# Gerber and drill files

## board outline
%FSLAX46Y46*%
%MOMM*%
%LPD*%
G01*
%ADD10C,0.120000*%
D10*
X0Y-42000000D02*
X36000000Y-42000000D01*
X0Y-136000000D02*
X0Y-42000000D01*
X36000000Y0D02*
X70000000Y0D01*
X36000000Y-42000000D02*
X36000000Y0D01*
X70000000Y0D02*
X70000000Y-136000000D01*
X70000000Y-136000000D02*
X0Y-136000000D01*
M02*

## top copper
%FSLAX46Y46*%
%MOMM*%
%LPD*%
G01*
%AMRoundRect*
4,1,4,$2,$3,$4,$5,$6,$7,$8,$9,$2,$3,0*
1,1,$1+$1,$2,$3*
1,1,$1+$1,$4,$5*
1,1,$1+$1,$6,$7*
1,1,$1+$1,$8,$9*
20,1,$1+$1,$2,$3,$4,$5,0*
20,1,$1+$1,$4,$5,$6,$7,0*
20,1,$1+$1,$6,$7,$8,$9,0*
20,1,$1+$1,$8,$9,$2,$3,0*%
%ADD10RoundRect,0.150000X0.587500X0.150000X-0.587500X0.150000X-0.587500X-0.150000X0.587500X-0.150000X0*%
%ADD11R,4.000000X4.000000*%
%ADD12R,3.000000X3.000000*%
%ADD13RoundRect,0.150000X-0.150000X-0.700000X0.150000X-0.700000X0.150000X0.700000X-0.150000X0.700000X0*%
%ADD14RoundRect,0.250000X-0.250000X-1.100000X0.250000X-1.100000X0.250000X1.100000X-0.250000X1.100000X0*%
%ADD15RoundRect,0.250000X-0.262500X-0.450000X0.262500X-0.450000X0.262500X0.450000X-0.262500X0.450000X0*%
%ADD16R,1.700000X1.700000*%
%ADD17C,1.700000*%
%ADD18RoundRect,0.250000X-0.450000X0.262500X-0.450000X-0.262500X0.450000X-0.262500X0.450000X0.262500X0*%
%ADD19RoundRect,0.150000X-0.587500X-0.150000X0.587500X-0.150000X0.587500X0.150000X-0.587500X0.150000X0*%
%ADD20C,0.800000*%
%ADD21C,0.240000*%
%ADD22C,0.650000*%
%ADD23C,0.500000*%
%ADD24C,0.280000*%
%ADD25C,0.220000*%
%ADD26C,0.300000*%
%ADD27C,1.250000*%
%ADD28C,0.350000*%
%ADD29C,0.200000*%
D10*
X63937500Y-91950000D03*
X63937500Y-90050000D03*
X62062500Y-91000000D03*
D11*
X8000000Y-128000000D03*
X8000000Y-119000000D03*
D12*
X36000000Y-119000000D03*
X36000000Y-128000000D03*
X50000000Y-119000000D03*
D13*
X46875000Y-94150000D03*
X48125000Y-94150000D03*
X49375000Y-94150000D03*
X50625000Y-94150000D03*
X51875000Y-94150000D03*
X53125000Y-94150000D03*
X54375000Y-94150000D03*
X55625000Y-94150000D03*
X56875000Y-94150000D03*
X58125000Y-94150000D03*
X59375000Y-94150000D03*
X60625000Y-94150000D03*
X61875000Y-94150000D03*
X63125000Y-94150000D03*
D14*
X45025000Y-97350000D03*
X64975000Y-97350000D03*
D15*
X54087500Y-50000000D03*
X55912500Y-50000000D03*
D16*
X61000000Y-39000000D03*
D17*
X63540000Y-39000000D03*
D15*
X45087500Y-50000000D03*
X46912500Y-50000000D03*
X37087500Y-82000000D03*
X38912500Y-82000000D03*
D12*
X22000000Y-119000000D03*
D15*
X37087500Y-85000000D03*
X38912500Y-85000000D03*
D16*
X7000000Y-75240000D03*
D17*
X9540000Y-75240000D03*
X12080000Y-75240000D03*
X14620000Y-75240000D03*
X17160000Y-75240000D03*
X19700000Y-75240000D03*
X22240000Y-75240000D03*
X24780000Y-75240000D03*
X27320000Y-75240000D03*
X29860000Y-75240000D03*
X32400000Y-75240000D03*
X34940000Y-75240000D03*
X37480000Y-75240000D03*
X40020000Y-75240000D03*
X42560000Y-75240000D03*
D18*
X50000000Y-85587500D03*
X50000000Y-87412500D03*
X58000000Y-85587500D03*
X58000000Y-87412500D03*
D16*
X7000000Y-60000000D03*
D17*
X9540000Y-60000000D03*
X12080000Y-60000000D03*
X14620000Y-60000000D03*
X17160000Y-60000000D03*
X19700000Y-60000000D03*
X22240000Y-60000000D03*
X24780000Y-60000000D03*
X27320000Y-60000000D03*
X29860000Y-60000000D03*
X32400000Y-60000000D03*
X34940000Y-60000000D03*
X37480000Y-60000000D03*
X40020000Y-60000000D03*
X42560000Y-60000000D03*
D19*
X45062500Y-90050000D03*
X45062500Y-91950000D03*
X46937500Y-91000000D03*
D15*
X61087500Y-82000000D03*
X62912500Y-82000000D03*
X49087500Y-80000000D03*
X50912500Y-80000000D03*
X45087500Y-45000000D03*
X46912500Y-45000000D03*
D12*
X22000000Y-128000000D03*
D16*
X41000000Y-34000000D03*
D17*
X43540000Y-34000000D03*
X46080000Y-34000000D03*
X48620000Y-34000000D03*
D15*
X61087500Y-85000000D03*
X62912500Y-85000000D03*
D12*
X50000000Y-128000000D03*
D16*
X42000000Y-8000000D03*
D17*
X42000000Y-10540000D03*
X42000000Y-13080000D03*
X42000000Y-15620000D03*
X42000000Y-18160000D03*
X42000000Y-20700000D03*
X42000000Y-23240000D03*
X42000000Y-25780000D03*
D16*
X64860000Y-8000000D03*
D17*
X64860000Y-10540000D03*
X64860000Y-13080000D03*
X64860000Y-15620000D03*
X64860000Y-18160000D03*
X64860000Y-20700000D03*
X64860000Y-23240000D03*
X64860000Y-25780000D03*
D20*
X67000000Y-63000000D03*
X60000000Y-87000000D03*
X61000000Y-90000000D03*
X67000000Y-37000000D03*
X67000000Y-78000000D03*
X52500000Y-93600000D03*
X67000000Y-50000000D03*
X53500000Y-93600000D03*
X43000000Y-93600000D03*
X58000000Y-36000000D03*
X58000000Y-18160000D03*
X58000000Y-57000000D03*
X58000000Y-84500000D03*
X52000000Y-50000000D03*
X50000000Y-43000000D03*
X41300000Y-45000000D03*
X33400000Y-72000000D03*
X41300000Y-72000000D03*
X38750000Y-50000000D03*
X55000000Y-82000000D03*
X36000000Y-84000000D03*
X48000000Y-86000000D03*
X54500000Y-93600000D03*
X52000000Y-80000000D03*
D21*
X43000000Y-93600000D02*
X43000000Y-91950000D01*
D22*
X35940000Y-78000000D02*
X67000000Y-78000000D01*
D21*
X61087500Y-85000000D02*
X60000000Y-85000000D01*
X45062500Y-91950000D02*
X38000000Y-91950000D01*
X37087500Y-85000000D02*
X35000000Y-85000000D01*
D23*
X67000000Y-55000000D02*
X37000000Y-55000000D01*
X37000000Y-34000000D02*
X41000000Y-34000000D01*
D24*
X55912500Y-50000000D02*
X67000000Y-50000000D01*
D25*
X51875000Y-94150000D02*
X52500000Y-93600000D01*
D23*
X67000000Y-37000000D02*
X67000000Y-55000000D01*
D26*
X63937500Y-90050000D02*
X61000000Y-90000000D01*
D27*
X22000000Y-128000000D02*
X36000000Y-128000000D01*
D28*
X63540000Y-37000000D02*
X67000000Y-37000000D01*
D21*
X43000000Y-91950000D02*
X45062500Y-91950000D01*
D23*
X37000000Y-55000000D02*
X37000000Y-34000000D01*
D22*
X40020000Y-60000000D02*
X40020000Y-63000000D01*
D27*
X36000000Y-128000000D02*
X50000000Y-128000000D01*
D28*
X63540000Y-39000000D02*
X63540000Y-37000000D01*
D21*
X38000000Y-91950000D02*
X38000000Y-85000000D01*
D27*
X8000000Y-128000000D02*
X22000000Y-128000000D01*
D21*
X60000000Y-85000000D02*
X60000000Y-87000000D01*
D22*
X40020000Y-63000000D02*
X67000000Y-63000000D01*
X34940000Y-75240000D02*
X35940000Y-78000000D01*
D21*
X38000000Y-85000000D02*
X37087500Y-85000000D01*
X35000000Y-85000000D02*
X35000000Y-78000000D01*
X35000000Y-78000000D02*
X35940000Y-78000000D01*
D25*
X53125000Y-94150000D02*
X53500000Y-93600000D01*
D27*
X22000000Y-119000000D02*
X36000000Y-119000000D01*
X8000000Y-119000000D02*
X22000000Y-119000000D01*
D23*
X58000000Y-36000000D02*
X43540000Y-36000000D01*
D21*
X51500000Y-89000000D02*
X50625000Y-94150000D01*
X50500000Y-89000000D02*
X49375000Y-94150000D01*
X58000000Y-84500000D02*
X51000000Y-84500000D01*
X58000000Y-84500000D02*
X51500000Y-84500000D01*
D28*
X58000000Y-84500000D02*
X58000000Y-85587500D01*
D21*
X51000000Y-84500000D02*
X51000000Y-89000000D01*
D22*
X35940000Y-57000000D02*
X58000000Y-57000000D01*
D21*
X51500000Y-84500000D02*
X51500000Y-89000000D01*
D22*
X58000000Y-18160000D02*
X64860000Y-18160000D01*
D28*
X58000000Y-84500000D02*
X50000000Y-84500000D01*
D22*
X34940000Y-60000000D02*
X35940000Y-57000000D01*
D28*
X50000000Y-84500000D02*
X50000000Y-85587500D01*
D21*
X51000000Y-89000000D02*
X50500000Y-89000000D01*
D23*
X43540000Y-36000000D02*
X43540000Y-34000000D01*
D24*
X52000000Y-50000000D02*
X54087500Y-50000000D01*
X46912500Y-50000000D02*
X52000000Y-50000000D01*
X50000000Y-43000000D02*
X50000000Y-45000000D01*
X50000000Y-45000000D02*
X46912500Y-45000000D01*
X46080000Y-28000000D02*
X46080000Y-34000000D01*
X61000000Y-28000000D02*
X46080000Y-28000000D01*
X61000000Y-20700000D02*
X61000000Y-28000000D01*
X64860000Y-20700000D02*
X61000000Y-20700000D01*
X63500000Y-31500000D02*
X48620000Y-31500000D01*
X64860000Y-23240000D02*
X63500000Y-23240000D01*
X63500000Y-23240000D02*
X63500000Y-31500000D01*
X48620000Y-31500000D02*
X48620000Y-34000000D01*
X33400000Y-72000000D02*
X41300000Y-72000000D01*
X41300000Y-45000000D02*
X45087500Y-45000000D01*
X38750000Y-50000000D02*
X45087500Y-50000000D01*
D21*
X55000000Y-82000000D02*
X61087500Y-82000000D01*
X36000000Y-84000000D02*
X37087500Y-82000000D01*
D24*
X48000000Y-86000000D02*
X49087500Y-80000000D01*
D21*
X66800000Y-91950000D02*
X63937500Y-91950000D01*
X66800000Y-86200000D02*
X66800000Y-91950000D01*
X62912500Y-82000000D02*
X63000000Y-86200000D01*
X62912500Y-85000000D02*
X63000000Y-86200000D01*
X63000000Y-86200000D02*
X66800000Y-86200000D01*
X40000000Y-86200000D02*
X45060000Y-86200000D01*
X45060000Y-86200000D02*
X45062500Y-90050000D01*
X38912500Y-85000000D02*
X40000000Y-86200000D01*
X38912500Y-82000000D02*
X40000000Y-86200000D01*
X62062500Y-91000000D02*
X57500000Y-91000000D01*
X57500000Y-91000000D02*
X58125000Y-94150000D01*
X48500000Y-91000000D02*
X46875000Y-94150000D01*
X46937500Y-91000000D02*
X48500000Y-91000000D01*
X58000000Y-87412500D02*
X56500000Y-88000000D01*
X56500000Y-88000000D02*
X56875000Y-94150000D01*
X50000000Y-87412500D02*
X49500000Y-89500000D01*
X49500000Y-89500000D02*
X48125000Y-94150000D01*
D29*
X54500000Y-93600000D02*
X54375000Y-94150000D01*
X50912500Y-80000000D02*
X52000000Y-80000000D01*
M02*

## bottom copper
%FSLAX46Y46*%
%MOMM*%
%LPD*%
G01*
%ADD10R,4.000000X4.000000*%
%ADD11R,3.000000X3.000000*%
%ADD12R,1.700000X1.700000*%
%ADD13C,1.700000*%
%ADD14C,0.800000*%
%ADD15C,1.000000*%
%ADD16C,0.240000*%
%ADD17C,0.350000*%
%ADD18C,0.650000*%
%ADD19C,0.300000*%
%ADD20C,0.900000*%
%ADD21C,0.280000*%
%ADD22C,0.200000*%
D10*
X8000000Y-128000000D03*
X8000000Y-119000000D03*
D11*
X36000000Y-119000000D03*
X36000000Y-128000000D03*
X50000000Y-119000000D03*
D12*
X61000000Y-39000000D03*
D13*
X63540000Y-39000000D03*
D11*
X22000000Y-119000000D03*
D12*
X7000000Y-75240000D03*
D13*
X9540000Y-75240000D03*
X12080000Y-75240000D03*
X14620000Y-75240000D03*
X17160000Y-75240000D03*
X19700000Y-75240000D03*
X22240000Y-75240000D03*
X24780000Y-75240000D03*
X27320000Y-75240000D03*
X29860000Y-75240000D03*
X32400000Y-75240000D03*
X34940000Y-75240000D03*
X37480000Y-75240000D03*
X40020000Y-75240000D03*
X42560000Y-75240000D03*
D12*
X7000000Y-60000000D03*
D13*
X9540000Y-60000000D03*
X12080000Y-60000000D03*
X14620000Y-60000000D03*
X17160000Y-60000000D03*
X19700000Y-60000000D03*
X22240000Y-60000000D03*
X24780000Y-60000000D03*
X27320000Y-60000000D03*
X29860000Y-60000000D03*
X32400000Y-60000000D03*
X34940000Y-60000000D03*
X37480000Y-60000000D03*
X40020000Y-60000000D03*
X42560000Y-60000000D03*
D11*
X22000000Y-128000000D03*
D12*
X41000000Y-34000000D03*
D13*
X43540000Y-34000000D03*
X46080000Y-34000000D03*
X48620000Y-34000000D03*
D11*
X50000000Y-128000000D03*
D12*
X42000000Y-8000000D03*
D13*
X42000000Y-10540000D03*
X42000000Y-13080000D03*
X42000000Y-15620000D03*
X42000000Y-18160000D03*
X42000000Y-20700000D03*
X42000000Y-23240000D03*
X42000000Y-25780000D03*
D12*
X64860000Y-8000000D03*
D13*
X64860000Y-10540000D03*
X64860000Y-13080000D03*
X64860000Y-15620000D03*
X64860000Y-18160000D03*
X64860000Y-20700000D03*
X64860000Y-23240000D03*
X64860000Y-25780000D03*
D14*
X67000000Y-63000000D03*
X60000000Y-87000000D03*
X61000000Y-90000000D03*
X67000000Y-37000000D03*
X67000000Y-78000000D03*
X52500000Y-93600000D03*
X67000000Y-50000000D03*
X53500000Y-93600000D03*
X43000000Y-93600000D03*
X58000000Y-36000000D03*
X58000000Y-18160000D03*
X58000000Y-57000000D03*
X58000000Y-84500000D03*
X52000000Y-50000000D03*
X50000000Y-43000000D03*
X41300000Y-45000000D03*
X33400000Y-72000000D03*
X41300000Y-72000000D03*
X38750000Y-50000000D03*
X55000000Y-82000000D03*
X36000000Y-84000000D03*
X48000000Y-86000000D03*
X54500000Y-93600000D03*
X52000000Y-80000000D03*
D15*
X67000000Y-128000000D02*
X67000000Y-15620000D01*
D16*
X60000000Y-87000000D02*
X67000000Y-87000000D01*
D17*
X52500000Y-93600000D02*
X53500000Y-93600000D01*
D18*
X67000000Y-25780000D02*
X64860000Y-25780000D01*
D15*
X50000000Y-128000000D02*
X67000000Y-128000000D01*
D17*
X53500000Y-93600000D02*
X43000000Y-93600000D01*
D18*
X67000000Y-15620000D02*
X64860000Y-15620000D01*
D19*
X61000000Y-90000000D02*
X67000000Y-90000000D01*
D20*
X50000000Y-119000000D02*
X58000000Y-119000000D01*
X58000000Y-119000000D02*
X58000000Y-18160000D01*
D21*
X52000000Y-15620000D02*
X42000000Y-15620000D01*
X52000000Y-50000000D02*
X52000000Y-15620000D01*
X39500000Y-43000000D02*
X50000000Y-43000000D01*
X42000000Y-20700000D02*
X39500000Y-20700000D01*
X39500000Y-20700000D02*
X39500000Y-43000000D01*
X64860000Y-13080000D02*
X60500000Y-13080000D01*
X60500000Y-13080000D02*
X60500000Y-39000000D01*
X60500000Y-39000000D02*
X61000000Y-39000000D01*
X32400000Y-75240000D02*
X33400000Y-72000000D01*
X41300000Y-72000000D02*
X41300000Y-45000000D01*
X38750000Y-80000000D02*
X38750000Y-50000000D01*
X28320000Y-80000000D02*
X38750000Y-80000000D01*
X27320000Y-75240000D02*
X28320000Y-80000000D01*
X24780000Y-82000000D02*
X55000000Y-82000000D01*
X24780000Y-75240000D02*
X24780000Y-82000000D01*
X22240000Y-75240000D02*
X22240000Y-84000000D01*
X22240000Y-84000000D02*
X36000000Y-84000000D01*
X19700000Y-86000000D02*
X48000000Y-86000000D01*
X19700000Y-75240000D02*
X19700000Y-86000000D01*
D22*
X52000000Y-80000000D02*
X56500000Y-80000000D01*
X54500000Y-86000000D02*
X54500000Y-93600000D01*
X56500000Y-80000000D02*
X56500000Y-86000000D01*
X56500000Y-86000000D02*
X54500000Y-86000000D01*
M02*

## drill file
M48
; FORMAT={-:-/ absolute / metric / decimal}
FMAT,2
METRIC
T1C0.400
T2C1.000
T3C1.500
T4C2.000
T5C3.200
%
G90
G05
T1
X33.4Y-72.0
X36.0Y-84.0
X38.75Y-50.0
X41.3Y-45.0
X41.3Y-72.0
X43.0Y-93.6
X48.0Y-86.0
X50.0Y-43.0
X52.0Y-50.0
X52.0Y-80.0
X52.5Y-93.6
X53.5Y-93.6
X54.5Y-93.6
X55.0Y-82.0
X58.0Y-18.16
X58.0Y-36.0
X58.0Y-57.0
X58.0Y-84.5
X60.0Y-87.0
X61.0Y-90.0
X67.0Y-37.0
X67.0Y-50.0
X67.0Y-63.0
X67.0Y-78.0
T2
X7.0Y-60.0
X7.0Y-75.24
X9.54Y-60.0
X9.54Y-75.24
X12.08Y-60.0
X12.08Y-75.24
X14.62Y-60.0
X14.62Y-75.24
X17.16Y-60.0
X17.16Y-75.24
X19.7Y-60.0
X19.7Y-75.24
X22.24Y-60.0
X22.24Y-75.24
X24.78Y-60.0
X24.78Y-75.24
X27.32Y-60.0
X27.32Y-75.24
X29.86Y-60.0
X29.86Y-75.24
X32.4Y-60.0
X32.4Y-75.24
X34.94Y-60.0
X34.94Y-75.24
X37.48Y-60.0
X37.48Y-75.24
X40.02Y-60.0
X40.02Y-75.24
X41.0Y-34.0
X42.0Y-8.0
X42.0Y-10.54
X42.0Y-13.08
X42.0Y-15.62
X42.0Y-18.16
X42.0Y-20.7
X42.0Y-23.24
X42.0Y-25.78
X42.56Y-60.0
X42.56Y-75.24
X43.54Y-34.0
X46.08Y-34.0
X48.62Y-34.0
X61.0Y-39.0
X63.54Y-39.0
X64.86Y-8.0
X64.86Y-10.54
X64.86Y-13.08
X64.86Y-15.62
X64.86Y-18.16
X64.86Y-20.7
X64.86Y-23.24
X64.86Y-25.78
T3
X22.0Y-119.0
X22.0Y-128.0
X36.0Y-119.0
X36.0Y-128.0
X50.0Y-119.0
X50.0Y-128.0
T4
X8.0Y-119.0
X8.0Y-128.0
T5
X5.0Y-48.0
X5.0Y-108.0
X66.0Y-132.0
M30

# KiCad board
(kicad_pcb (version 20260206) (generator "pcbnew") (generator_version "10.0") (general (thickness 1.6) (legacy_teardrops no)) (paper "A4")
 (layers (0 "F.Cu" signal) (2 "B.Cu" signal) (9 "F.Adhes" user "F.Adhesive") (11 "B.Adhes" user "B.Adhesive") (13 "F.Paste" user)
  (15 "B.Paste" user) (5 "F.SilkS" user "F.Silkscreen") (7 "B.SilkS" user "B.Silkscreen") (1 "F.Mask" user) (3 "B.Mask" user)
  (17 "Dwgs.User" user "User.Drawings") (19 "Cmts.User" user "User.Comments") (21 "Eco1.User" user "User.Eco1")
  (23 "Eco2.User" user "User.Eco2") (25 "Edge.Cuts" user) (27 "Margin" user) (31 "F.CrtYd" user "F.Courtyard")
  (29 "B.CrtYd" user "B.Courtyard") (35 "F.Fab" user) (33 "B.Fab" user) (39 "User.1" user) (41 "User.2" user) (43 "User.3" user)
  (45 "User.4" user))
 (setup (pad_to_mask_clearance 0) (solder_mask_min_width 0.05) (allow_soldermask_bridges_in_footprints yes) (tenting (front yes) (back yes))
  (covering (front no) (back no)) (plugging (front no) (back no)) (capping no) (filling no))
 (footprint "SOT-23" (layer "F.Cu") (at 63 91 180)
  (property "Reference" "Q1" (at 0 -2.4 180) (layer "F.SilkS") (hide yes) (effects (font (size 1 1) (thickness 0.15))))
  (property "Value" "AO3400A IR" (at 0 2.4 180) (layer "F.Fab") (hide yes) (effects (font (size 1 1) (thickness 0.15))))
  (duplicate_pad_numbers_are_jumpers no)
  (pad "1" smd roundrect (at -0.9375 -0.95 180) (size 1.475 0.6) (layers "F.Cu" "F.Mask" "F.Paste") (roundrect_rratio 0.25) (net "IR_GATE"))
  (pad "2" smd roundrect (at -0.9375 0.95 180) (size 1.475 0.6) (layers "F.Cu" "F.Mask" "F.Paste") (roundrect_rratio 0.25) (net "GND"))
  (pad "3" smd roundrect (at 0.9375 0 180) (size 1.475 0.6) (layers "F.Cu" "F.Mask" "F.Paste") (roundrect_rratio 0.25) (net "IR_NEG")))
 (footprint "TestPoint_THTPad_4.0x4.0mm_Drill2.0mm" (layer "F.Cu") (at 8 128)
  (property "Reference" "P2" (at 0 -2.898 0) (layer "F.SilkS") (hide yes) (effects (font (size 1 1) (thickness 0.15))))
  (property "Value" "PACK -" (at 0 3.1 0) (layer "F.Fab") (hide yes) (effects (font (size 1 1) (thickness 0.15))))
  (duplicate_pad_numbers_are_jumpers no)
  (pad "1" thru_hole rect (at 0 0) (size 4 4) (drill 2) (layers "*.Cu" "*.Mask") (remove_unused_layers no) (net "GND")))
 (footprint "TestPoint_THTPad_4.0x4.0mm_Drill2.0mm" (layer "F.Cu") (at 8 119)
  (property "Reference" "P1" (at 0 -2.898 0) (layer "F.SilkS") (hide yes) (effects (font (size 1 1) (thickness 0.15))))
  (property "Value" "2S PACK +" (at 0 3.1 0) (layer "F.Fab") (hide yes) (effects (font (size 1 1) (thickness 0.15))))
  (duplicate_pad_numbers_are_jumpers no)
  (pad "1" thru_hole rect (at 0 0) (size 4 4) (drill 2) (layers "*.Cu" "*.Mask") (remove_unused_layers no) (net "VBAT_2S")))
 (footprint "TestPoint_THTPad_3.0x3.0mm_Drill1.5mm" (layer "F.Cu") (at 36 119)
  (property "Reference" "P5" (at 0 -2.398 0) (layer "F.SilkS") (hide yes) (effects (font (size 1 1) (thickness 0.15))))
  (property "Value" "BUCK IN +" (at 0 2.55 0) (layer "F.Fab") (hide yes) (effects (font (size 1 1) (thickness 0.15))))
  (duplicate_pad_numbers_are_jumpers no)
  (pad "1" thru_hole rect (at 0 0) (size 3 3) (drill 1.5) (layers "*.Cu" "*.Mask") (remove_unused_layers no) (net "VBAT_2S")))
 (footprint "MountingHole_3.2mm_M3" (layer "F.Cu") (at 5 48)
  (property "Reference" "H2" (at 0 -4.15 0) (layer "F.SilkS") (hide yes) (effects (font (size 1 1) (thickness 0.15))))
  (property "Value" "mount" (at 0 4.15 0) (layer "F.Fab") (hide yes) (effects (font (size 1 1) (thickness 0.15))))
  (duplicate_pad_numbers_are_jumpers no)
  (pad "" np_thru_hole circle (at 0 0) (size 3.2 3.2) (drill 3.2) (layers "*.Cu" "*.Mask")))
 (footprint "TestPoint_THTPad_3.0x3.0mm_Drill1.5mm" (layer "F.Cu") (at 36 128)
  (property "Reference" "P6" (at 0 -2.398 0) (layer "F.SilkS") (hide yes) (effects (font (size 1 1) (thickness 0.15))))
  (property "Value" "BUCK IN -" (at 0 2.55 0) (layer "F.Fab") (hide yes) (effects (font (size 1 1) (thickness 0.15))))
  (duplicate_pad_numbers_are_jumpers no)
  (pad "1" thru_hole rect (at 0 0) (size 3 3) (drill 1.5) (layers "*.Cu" "*.Mask") (remove_unused_layers no) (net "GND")))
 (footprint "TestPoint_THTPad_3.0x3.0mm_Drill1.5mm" (layer "F.Cu") (at 50 119)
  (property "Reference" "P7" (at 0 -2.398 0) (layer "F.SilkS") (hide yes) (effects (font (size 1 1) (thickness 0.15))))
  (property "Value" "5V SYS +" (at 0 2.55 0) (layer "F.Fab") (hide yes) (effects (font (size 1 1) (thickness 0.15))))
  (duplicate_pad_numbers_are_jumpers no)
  (pad "1" thru_hole rect (at 0 0) (size 3 3) (drill 1.5) (layers "*.Cu" "*.Mask") (remove_unused_layers no) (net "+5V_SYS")))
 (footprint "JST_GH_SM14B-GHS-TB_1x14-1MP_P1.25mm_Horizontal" (layer "F.Cu") (at 55 96)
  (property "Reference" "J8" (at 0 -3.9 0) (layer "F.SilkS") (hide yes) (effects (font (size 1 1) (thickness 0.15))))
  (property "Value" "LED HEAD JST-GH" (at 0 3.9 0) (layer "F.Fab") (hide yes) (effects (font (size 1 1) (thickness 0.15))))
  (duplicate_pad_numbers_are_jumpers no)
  (pad "1" smd roundrect (at -8.125 -1.85) (size 0.6 1.7) (layers "F.Cu" "F.Mask" "F.Paste") (roundrect_rratio 0.25) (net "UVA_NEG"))
  (pad "2" smd roundrect (at -6.875 -1.85) (size 0.6 1.7) (layers "F.Cu" "F.Mask" "F.Paste") (roundrect_rratio 0.25) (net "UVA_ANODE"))
  (pad "3" smd roundrect (at -5.625 -1.85) (size 0.6 1.7) (layers "F.Cu" "F.Mask" "F.Paste") (roundrect_rratio 0.25) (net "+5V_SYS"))
  (pad "4" smd roundrect (at -4.375 -1.85) (size 0.6 1.7) (layers "F.Cu" "F.Mask" "F.Paste") (roundrect_rratio 0.25) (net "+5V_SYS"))
  (pad "5" smd roundrect (at -3.125 -1.85) (size 0.6 1.7) (layers "F.Cu" "F.Mask" "F.Paste") (roundrect_rratio 0.25) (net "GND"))
  (pad "6" smd roundrect (at -1.875 -1.85) (size 0.6 1.7) (layers "F.Cu" "F.Mask" "F.Paste") (roundrect_rratio 0.25) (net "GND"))
  (pad "7" smd roundrect (at -0.625 -1.85) (size 0.6 1.7) (layers "F.Cu" "F.Mask" "F.Paste") (roundrect_rratio 0.25) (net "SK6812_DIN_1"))
  (pad "8" smd roundrect (at 0.625 -1.85) (size 0.6 1.7) (layers "F.Cu" "F.Mask" "F.Paste") (roundrect_rratio 0.25))
  (pad "9" smd roundrect (at 1.875 -1.85) (size 0.6 1.7) (layers "F.Cu" "F.Mask" "F.Paste") (roundrect_rratio 0.25) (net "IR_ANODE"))
  (pad "10" smd roundrect (at 3.125 -1.85) (size 0.6 1.7) (layers "F.Cu" "F.Mask" "F.Paste") (roundrect_rratio 0.25) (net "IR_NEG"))
  (pad "11" smd roundrect (at 4.375 -1.85) (size 0.6 1.7) (layers "F.Cu" "F.Mask" "F.Paste") (roundrect_rratio 0.25))
  (pad "12" smd roundrect (at 5.625 -1.85) (size 0.6 1.7) (layers "F.Cu" "F.Mask" "F.Paste") (roundrect_rratio 0.25))
  (pad "13" smd roundrect (at 6.875 -1.85) (size 0.6 1.7) (layers "F.Cu" "F.Mask" "F.Paste") (roundrect_rratio 0.25))
  (pad "14" smd roundrect (at 8.125 -1.85) (size 0.6 1.7) (layers "F.Cu" "F.Mask" "F.Paste") (roundrect_rratio 0.25))
  (pad "MP" smd roundrect (at -9.975 1.35) (size 1 2.7) (layers "F.Cu" "F.Mask" "F.Paste") (roundrect_rratio 0.25))
  (pad "MP" smd roundrect (at 9.975 1.35) (size 1 2.7) (layers "F.Cu" "F.Mask" "F.Paste") (roundrect_rratio 0.25)))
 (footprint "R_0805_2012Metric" (layer "F.Cu") (at 55 50)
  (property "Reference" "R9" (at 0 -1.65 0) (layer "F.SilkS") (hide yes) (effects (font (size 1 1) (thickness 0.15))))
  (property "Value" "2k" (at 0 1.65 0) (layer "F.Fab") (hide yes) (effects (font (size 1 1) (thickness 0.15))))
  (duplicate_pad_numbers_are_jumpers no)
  (pad "1" smd roundrect (at -0.9125 0) (size 1.025 1.4) (layers "F.Cu" "F.Mask" "F.Paste") (roundrect_rratio 0.243902)
   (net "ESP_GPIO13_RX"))
  (pad "2" smd roundrect (at 0.9125 0) (size 1.025 1.4) (layers "F.Cu" "F.Mask" "F.Paste") (roundrect_rratio 0.243902) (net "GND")))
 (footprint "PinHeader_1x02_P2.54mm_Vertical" (layer "F.Cu") (at 61 39 90)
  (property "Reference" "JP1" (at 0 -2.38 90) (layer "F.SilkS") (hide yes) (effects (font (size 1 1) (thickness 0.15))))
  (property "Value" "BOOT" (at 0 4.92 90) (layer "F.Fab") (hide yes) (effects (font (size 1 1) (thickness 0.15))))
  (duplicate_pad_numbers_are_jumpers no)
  (pad "1" thru_hole rect (at 0 0 90) (size 1.7 1.7) (drill 1) (layers "*.Cu" "*.Mask") (remove_unused_layers no) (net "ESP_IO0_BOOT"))
  (pad "2" thru_hole circle (at 0 2.54 90) (size 1.7 1.7) (drill 1) (layers "*.Cu" "*.Mask") (remove_unused_layers no) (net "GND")))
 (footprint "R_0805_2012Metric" (layer "F.Cu") (at 46 50)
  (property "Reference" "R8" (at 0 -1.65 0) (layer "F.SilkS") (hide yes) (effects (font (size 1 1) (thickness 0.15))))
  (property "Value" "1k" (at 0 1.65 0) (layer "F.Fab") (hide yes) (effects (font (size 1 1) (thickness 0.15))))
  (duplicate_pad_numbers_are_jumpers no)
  (pad "1" smd roundrect (at -0.9125 0) (size 1.025 1.4) (layers "F.Cu" "F.Mask" "F.Paste") (roundrect_rratio 0.243902) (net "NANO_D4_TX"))
  (pad "2" smd roundrect (at 0.9125 0) (size 1.025 1.4) (layers "F.Cu" "F.Mask" "F.Paste") (roundrect_rratio 0.243902) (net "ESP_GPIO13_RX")))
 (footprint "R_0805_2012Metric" (layer "F.Cu") (at 38 82)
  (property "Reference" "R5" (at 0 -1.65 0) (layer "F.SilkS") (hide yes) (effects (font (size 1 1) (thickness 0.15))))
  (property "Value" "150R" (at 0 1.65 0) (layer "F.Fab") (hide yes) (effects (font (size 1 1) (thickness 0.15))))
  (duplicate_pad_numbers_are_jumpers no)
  (pad "1" smd roundrect (at -0.9125 0) (size 1.025 1.4) (layers "F.Cu" "F.Mask" "F.Paste") (roundrect_rratio 0.243902)
   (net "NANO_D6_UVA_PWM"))
  (pad "2" smd roundrect (at 0.9125 0) (size 1.025 1.4) (layers "F.Cu" "F.Mask" "F.Paste") (roundrect_rratio 0.243902) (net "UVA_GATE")))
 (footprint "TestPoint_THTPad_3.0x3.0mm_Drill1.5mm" (layer "F.Cu") (at 22 119)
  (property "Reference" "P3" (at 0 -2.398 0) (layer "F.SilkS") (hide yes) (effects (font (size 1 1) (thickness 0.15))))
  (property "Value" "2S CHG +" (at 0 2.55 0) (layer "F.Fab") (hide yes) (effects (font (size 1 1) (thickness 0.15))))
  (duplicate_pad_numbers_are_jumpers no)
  (pad "1" thru_hole rect (at 0 0) (size 3 3) (drill 1.5) (layers "*.Cu" "*.Mask") (remove_unused_layers no) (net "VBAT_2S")))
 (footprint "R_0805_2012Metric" (layer "F.Cu") (at 38 85)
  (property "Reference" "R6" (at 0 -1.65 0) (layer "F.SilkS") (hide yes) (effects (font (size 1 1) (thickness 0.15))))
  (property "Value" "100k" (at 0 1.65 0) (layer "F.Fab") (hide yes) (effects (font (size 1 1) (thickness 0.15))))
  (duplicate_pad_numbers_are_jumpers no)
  (pad "1" smd roundrect (at -0.9125 0) (size 1.025 1.4) (layers "F.Cu" "F.Mask" "F.Paste") (roundrect_rratio 0.243902) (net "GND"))
  (pad "2" smd roundrect (at 0.9125 0) (size 1.025 1.4) (layers "F.Cu" "F.Mask" "F.Paste") (roundrect_rratio 0.243902) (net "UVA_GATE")))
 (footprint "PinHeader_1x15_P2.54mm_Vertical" (layer "F.Cu") (at 7 75.24 90)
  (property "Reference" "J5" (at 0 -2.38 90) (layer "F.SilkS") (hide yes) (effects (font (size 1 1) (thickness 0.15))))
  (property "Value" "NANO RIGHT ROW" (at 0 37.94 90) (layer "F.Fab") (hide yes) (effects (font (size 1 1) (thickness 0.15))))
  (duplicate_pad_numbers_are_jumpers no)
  (pad "1" thru_hole rect (at 0 0 90) (size 1.7 1.7) (drill 1) (layers "*.Cu" "*.Mask") (remove_unused_layers no))
  (pad "2" thru_hole circle (at 0 2.54 90) (size 1.7 1.7) (drill 1) (layers "*.Cu" "*.Mask") (remove_unused_layers no))
  (pad "3" thru_hole circle (at 0 5.08 90) (size 1.7 1.7) (drill 1) (layers "*.Cu" "*.Mask") (remove_unused_layers no))
  (pad "4" thru_hole circle (at 0 7.62 90) (size 1.7 1.7) (drill 1) (layers "*.Cu" "*.Mask") (remove_unused_layers no))
  (pad "5" thru_hole circle (at 0 10.16 90) (size 1.7 1.7) (drill 1) (layers "*.Cu" "*.Mask") (remove_unused_layers no)
   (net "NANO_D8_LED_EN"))
  (pad "6" thru_hole circle (at 0 12.7 90) (size 1.7 1.7) (drill 1) (layers "*.Cu" "*.Mask") (remove_unused_layers no)
   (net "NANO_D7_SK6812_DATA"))
  (pad "7" thru_hole circle (at 0 15.24 90) (size 1.7 1.7) (drill 1) (layers "*.Cu" "*.Mask") (remove_unused_layers no)
   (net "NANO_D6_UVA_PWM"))
  (pad "8" thru_hole circle (at 0 17.78 90) (size 1.7 1.7) (drill 1) (layers "*.Cu" "*.Mask") (remove_unused_layers no)
   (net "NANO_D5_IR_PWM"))
  (pad "9" thru_hole circle (at 0 20.32 90) (size 1.7 1.7) (drill 1) (layers "*.Cu" "*.Mask") (remove_unused_layers no) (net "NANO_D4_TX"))
  (pad "10" thru_hole circle (at 0 22.86 90) (size 1.7 1.7) (drill 1) (layers "*.Cu" "*.Mask") (remove_unused_layers no))
  (pad "11" thru_hole circle (at 0 25.4 90) (size 1.7 1.7) (drill 1) (layers "*.Cu" "*.Mask") (remove_unused_layers no) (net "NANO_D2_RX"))
  (pad "12" thru_hole circle (at 0 27.94 90) (size 1.7 1.7) (drill 1) (layers "*.Cu" "*.Mask") (remove_unused_layers no) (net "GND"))
  (pad "13" thru_hole circle (at 0 30.48 90) (size 1.7 1.7) (drill 1) (layers "*.Cu" "*.Mask") (remove_unused_layers no))
  (pad "14" thru_hole circle (at 0 33.02 90) (size 1.7 1.7) (drill 1) (layers "*.Cu" "*.Mask") (remove_unused_layers no))
  (pad "15" thru_hole circle (at 0 35.56 90) (size 1.7 1.7) (drill 1) (layers "*.Cu" "*.Mask") (remove_unused_layers no)))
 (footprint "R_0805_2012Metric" (layer "F.Cu") (at 50 86.5 -90)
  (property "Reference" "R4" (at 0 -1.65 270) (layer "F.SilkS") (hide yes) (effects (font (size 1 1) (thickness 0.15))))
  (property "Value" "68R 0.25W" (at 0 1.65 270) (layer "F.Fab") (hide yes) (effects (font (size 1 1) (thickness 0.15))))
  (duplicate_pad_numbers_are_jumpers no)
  (pad "1" smd roundrect (at -0.9125 0 270) (size 1.025 1.4) (layers "F.Cu" "F.Mask" "F.Paste") (roundrect_rratio 0.243902) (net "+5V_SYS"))
  (pad "2" smd roundrect (at 0.9125 0 270) (size 1.025 1.4) (layers "F.Cu" "F.Mask" "F.Paste") (roundrect_rratio 0.243902) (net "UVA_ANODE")))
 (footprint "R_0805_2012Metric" (layer "F.Cu") (at 58 86.5 -90)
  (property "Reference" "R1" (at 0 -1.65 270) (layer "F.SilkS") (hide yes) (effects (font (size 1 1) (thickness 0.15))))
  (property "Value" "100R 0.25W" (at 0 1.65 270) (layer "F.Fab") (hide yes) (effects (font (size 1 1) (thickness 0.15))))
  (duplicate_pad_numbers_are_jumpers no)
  (pad "1" smd roundrect (at -0.9125 0 270) (size 1.025 1.4) (layers "F.Cu" "F.Mask" "F.Paste") (roundrect_rratio 0.243902) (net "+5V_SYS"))
  (pad "2" smd roundrect (at 0.9125 0 270) (size 1.025 1.4) (layers "F.Cu" "F.Mask" "F.Paste") (roundrect_rratio 0.243902) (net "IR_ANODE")))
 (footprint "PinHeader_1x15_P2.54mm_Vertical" (layer "F.Cu") (at 7 60 90)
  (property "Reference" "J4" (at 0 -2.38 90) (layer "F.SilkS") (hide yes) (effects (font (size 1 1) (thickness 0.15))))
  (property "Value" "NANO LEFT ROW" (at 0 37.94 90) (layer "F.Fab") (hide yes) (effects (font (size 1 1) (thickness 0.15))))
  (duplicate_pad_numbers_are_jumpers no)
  (pad "1" thru_hole rect (at 0 0 90) (size 1.7 1.7) (drill 1) (layers "*.Cu" "*.Mask") (remove_unused_layers no))
  (pad "2" thru_hole circle (at 0 2.54 90) (size 1.7 1.7) (drill 1) (layers "*.Cu" "*.Mask") (remove_unused_layers no))
  (pad "3" thru_hole circle (at 0 5.08 90) (size 1.7 1.7) (drill 1) (layers "*.Cu" "*.Mask") (remove_unused_layers no))
  (pad "4" thru_hole circle (at 0 7.62 90) (size 1.7 1.7) (drill 1) (layers "*.Cu" "*.Mask") (remove_unused_layers no))
  (pad "5" thru_hole circle (at 0 10.16 90) (size 1.7 1.7) (drill 1) (layers "*.Cu" "*.Mask") (remove_unused_layers no))
  (pad "6" thru_hole circle (at 0 12.7 90) (size 1.7 1.7) (drill 1) (layers "*.Cu" "*.Mask") (remove_unused_layers no))
  (pad "7" thru_hole circle (at 0 15.24 90) (size 1.7 1.7) (drill 1) (layers "*.Cu" "*.Mask") (remove_unused_layers no))
  (pad "8" thru_hole circle (at 0 17.78 90) (size 1.7 1.7) (drill 1) (layers "*.Cu" "*.Mask") (remove_unused_layers no))
  (pad "9" thru_hole circle (at 0 20.32 90) (size 1.7 1.7) (drill 1) (layers "*.Cu" "*.Mask") (remove_unused_layers no))
  (pad "10" thru_hole circle (at 0 22.86 90) (size 1.7 1.7) (drill 1) (layers "*.Cu" "*.Mask") (remove_unused_layers no))
  (pad "11" thru_hole circle (at 0 25.4 90) (size 1.7 1.7) (drill 1) (layers "*.Cu" "*.Mask") (remove_unused_layers no))
  (pad "12" thru_hole circle (at 0 27.94 90) (size 1.7 1.7) (drill 1) (layers "*.Cu" "*.Mask") (remove_unused_layers no) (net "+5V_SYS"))
  (pad "13" thru_hole circle (at 0 30.48 90) (size 1.7 1.7) (drill 1) (layers "*.Cu" "*.Mask") (remove_unused_layers no))
  (pad "14" thru_hole circle (at 0 33.02 90) (size 1.7 1.7) (drill 1) (layers "*.Cu" "*.Mask") (remove_unused_layers no) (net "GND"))
  (pad "15" thru_hole circle (at 0 35.56 90) (size 1.7 1.7) (drill 1) (layers "*.Cu" "*.Mask") (remove_unused_layers no)))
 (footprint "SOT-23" (layer "F.Cu") (at 46 91)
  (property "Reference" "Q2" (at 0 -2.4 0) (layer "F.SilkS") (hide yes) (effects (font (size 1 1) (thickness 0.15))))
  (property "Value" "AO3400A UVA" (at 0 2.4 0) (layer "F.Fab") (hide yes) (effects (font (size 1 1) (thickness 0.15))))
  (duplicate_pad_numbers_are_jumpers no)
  (pad "1" smd roundrect (at -0.9375 -0.95) (size 1.475 0.6) (layers "F.Cu" "F.Mask" "F.Paste") (roundrect_rratio 0.25) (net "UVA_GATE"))
  (pad "2" smd roundrect (at -0.9375 0.95) (size 1.475 0.6) (layers "F.Cu" "F.Mask" "F.Paste") (roundrect_rratio 0.25) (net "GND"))
  (pad "3" smd roundrect (at 0.9375 0) (size 1.475 0.6) (layers "F.Cu" "F.Mask" "F.Paste") (roundrect_rratio 0.25) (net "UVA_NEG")))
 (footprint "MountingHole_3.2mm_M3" (layer "F.Cu") (at 66 132)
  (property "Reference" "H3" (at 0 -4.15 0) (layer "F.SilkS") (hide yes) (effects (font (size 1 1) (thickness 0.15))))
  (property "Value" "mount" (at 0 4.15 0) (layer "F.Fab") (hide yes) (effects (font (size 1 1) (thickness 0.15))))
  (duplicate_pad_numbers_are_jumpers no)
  (pad "" np_thru_hole circle (at 0 0) (size 3.2 3.2) (drill 3.2) (layers "*.Cu" "*.Mask")))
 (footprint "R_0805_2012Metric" (layer "F.Cu") (at 62 82)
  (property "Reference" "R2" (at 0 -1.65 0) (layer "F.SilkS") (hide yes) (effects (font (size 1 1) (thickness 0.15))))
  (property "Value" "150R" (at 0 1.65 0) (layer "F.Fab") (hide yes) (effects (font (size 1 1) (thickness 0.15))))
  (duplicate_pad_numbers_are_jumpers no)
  (pad "1" smd roundrect (at -0.9125 0) (size 1.025 1.4) (layers "F.Cu" "F.Mask" "F.Paste") (roundrect_rratio 0.243902)
   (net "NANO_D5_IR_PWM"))
  (pad "2" smd roundrect (at 0.9125 0) (size 1.025 1.4) (layers "F.Cu" "F.Mask" "F.Paste") (roundrect_rratio 0.243902) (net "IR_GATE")))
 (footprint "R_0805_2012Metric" (layer "F.Cu") (at 50 80)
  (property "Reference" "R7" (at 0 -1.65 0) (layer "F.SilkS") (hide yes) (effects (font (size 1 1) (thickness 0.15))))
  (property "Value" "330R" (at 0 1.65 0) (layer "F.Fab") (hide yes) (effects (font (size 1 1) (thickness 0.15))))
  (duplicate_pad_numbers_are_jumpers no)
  (pad "1" smd roundrect (at -0.9125 0) (size 1.025 1.4) (layers "F.Cu" "F.Mask" "F.Paste") (roundrect_rratio 0.243902)
   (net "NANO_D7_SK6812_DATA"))
  (pad "2" smd roundrect (at 0.9125 0) (size 1.025 1.4) (layers "F.Cu" "F.Mask" "F.Paste") (roundrect_rratio 0.243902) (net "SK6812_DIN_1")))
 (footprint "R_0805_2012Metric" (layer "F.Cu") (at 46 45)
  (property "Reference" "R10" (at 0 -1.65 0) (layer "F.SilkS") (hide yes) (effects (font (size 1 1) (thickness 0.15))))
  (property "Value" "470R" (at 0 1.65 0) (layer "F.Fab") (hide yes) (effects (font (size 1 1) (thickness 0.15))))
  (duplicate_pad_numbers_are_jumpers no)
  (pad "1" smd roundrect (at -0.9125 0) (size 1.025 1.4) (layers "F.Cu" "F.Mask" "F.Paste") (roundrect_rratio 0.243902) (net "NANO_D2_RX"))
  (pad "2" smd roundrect (at 0.9125 0) (size 1.025 1.4) (layers "F.Cu" "F.Mask" "F.Paste") (roundrect_rratio 0.243902) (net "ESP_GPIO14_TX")))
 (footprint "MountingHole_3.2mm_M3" (layer "F.Cu") (at 5 108)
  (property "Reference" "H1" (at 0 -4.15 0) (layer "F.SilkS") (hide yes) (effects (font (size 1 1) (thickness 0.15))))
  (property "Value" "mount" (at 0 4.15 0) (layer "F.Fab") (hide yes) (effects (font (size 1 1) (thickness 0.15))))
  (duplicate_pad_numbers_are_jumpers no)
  (pad "" np_thru_hole circle (at 0 0) (size 3.2 3.2) (drill 3.2) (layers "*.Cu" "*.Mask")))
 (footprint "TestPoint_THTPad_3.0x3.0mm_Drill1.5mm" (layer "F.Cu") (at 22 128)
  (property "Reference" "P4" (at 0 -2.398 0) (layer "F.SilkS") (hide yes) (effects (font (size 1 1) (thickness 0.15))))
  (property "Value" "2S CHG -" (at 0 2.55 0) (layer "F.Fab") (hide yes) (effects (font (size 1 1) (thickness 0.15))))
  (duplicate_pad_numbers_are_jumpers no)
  (pad "1" thru_hole rect (at 0 0) (size 3 3) (drill 1.5) (layers "*.Cu" "*.Mask") (remove_unused_layers no) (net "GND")))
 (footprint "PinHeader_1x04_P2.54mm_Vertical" (layer "F.Cu") (at 41 34 90)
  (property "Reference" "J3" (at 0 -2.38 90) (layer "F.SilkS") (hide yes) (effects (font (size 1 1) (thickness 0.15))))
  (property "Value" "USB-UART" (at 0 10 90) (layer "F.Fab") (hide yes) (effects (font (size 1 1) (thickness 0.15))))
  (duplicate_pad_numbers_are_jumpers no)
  (pad "1" thru_hole rect (at 0 0 90) (size 1.7 1.7) (drill 1) (layers "*.Cu" "*.Mask") (remove_unused_layers no) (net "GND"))
  (pad "2" thru_hole circle (at 0 2.54 90) (size 1.7 1.7) (drill 1) (layers "*.Cu" "*.Mask") (remove_unused_layers no) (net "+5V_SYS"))
  (pad "3" thru_hole circle (at 0 5.08 90) (size 1.7 1.7) (drill 1) (layers "*.Cu" "*.Mask") (remove_unused_layers no) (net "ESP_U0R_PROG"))
  (pad "4" thru_hole circle (at 0 7.62 90) (size 1.7 1.7) (drill 1) (layers "*.Cu" "*.Mask") (remove_unused_layers no) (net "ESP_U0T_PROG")))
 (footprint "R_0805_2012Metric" (layer "F.Cu") (at 62 85)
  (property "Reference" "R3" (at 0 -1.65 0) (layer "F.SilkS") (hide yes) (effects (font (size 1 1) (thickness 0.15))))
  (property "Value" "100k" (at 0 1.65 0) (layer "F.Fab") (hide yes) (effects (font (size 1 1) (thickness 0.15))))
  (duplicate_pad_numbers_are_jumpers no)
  (pad "1" smd roundrect (at -0.9125 0) (size 1.025 1.4) (layers "F.Cu" "F.Mask" "F.Paste") (roundrect_rratio 0.243902) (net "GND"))
  (pad "2" smd roundrect (at 0.9125 0) (size 1.025 1.4) (layers "F.Cu" "F.Mask" "F.Paste") (roundrect_rratio 0.243902) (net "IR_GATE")))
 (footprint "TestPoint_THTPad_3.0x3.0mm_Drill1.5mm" (layer "F.Cu") (at 50 128)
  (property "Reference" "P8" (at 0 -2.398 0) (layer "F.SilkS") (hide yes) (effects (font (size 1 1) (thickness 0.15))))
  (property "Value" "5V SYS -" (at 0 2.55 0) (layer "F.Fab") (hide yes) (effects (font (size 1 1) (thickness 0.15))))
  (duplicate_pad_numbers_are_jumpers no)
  (pad "1" thru_hole rect (at 0 0) (size 3 3) (drill 1.5) (layers "*.Cu" "*.Mask") (remove_unused_layers no) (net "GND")))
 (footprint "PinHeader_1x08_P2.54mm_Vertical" (layer "F.Cu") (at 42 8)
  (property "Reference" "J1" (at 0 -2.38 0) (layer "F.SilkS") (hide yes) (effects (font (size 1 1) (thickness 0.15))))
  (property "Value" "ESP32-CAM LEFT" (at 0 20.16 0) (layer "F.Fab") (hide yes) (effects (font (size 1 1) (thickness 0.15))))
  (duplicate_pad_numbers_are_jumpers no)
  (pad "1" thru_hole rect (at 0 0) (size 1.7 1.7) (drill 1) (layers "*.Cu" "*.Mask") (remove_unused_layers no))
  (pad "2" thru_hole circle (at 0 2.54) (size 1.7 1.7) (drill 1) (layers "*.Cu" "*.Mask") (remove_unused_layers no))
  (pad "3" thru_hole circle (at 0 5.08) (size 1.7 1.7) (drill 1) (layers "*.Cu" "*.Mask") (remove_unused_layers no))
  (pad "4" thru_hole circle (at 0 7.62) (size 1.7 1.7) (drill 1) (layers "*.Cu" "*.Mask") (remove_unused_layers no) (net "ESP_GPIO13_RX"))
  (pad "5" thru_hole circle (at 0 10.16) (size 1.7 1.7) (drill 1) (layers "*.Cu" "*.Mask") (remove_unused_layers no))
  (pad "6" thru_hole circle (at 0 12.7) (size 1.7 1.7) (drill 1) (layers "*.Cu" "*.Mask") (remove_unused_layers no) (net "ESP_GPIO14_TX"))
  (pad "7" thru_hole circle (at 0 15.24) (size 1.7 1.7) (drill 1) (layers "*.Cu" "*.Mask") (remove_unused_layers no))
  (pad "8" thru_hole circle (at 0 17.78) (size 1.7 1.7) (drill 1) (layers "*.Cu" "*.Mask") (remove_unused_layers no)))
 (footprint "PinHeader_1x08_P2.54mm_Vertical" (layer "F.Cu") (at 64.86 8)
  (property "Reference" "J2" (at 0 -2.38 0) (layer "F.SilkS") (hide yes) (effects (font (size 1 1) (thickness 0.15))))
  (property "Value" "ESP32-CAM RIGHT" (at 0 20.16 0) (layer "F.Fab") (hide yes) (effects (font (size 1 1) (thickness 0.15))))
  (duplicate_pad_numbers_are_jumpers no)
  (pad "1" thru_hole rect (at 0 0) (size 1.7 1.7) (drill 1) (layers "*.Cu" "*.Mask") (remove_unused_layers no))
  (pad "2" thru_hole circle (at 0 2.54) (size 1.7 1.7) (drill 1) (layers "*.Cu" "*.Mask") (remove_unused_layers no))
  (pad "3" thru_hole circle (at 0 5.08) (size 1.7 1.7) (drill 1) (layers "*.Cu" "*.Mask") (remove_unused_layers no) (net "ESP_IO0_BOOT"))
  (pad "4" thru_hole circle (at 0 7.62) (size 1.7 1.7) (drill 1) (layers "*.Cu" "*.Mask") (remove_unused_layers no) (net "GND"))
  (pad "5" thru_hole circle (at 0 10.16) (size 1.7 1.7) (drill 1) (layers "*.Cu" "*.Mask") (remove_unused_layers no) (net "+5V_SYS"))
  (pad "6" thru_hole circle (at 0 12.7) (size 1.7 1.7) (drill 1) (layers "*.Cu" "*.Mask") (remove_unused_layers no) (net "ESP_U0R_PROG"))
  (pad "7" thru_hole circle (at 0 15.24) (size 1.7 1.7) (drill 1) (layers "*.Cu" "*.Mask") (remove_unused_layers no) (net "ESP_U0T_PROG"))
  (pad "8" thru_hole circle (at 0 17.78) (size 1.7 1.7) (drill 1) (layers "*.Cu" "*.Mask") (remove_unused_layers no) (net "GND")))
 (gr_line (start 0 42) (end 36 42) (stroke (width 0.12) (type default)) (layer "Edge.Cuts"))
 (gr_line (start 0 136) (end 0 42) (stroke (width 0.12) (type default)) (layer "Edge.Cuts"))
 (gr_line (start 36 0) (end 70 0) (stroke (width 0.12) (type default)) (layer "Edge.Cuts"))
 (gr_line (start 36 42) (end 36 0) (stroke (width 0.12) (type default)) (layer "Edge.Cuts"))
 (gr_line (start 70 0) (end 70 136) (stroke (width 0.12) (type default)) (layer "Edge.Cuts"))
 (gr_line (start 70 136) (end 0 136) (stroke (width 0.12) (type default)) (layer "Edge.Cuts"))
 (segment (start 43 93.6) (end 43 91.95) (width 0.24) (layer "F.Cu") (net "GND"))
 (segment (start 35.94 78) (end 67 78) (width 0.65) (layer "F.Cu") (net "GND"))
 (segment (start 61.0875 85) (end 60 85) (width 0.24) (layer "F.Cu") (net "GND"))
 (segment (start 45.0625 91.95) (end 38 91.95) (width 0.24) (layer "F.Cu") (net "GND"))
 (segment (start 37.0875 85) (end 35 85) (width 0.24) (layer "F.Cu") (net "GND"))
 (segment (start 67 55) (end 37 55) (width 0.5) (layer "F.Cu") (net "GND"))
 (segment (start 37 34) (end 41 34) (width 0.5) (layer "F.Cu") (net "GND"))
 (segment (start 55.9125 50) (end 67 50) (width 0.28) (layer "F.Cu") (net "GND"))
 (segment (start 51.875 94.15) (end 52.5 93.6) (width 0.22) (layer "F.Cu") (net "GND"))
 (segment (start 67 37) (end 67 55) (width 0.5) (layer "F.Cu") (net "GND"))
 (segment (start 63.9375 90.05) (end 61 90) (width 0.3) (layer "F.Cu") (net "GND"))
 (segment (start 22 128) (end 36 128) (width 1.25) (layer "F.Cu") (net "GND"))
 (segment (start 63.54 37) (end 67 37) (width 0.35) (layer "F.Cu") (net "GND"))
 (segment (start 43 91.95) (end 45.0625 91.95) (width 0.24) (layer "F.Cu") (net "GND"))
 (segment (start 37 55) (end 37 34) (width 0.5) (layer "F.Cu") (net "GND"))
 (segment (start 40.02 60) (end 40.02 63) (width 0.65) (layer "F.Cu") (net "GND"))
 (segment (start 36 128) (end 50 128) (width 1.25) (layer "F.Cu") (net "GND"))
 (segment (start 63.54 39) (end 63.54 37) (width 0.35) (layer "F.Cu") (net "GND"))
 (segment (start 38 91.95) (end 38 85) (width 0.24) (layer "F.Cu") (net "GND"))
 (segment (start 8 128) (end 22 128) (width 1.25) (layer "F.Cu") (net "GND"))
 (segment (start 60 85) (end 60 87) (width 0.24) (layer "F.Cu") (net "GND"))
 (segment (start 40.02 63) (end 67 63) (width 0.65) (layer "F.Cu") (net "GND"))
 (segment (start 34.94 75.24) (end 35.94 78) (width 0.65) (layer "F.Cu") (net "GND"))
 (segment (start 38 85) (end 37.0875 85) (width 0.24) (layer "F.Cu") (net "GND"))
 (segment (start 35 85) (end 35 78) (width 0.24) (layer "F.Cu") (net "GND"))
 (segment (start 35 78) (end 35.94 78) (width 0.24) (layer "F.Cu") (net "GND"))
 (segment (start 53.125 94.15) (end 53.5 93.6) (width 0.22) (layer "F.Cu") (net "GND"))
 (via (at 67 63) (size 0.8) (drill 0.4) (layers "F.Cu" "B.Cu") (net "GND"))
 (via (at 60 87) (size 0.8) (drill 0.4) (layers "F.Cu" "B.Cu") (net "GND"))
 (via (at 61 90) (size 0.8) (drill 0.4) (layers "F.Cu" "B.Cu") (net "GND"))
 (via (at 67 37) (size 0.8) (drill 0.4) (layers "F.Cu" "B.Cu") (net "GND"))
 (via (at 67 78) (size 0.8) (drill 0.4) (layers "F.Cu" "B.Cu") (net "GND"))
 (via (at 52.5 93.6) (size 0.8) (drill 0.4) (layers "F.Cu" "B.Cu") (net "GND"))
 (via (at 67 50) (size 0.8) (drill 0.4) (layers "F.Cu" "B.Cu") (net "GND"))
 (via (at 53.5 93.6) (size 0.8) (drill 0.4) (layers "F.Cu" "B.Cu") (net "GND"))
 (via (at 43 93.6) (size 0.8) (drill 0.4) (layers "F.Cu" "B.Cu") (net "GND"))
 (segment (start 67 128) (end 67 15.62) (width 1) (layer "B.Cu") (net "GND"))
 (segment (start 60 87) (end 67 87) (width 0.24) (layer "B.Cu") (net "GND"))
 (segment (start 52.5 93.6) (end 53.5 93.6) (width 0.35) (layer "B.Cu") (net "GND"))
 (segment (start 67 25.78) (end 64.86 25.78) (width 0.65) (layer "B.Cu") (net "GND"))
 (segment (start 50 128) (end 67 128) (width 1) (layer "B.Cu") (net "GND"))
 (segment (start 53.5 93.6) (end 43 93.6) (width 0.35) (layer "B.Cu") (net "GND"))
 (segment (start 67 15.62) (end 64.86 15.62) (width 0.65) (layer "B.Cu") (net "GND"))
 (segment (start 61 90) (end 67 90) (width 0.3) (layer "B.Cu") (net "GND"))
 (segment (start 22 119) (end 36 119) (width 1.25) (layer "F.Cu") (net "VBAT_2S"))
 (segment (start 8 119) (end 22 119) (width 1.25) (layer "F.Cu") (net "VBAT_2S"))
 (segment (start 58 36) (end 43.54 36) (width 0.5) (layer "F.Cu") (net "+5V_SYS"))
 (segment (start 51.5 89) (end 50.625 94.15) (width 0.24) (layer "F.Cu") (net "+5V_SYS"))
 (segment (start 50.5 89) (end 49.375 94.15) (width 0.24) (layer "F.Cu") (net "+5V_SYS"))
 (segment (start 58 84.5) (end 51 84.5) (width 0.24) (layer "F.Cu") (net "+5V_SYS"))
 (segment (start 58 84.5) (end 51.5 84.5) (width 0.24) (layer "F.Cu") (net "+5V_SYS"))
 (segment (start 58 84.5) (end 58 85.5875) (width 0.35) (layer "F.Cu") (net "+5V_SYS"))
 (segment (start 51 84.5) (end 51 89) (width 0.24) (layer "F.Cu") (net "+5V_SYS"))
 (segment (start 35.94 57) (end 58 57) (width 0.65) (layer "F.Cu") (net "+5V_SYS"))
 (segment (start 51.5 84.5) (end 51.5 89) (width 0.24) (layer "F.Cu") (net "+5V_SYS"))
 (segment (start 58 18.16) (end 64.86 18.16) (width 0.65) (layer "F.Cu") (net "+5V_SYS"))
 (segment (start 58 84.5) (end 50 84.5) (width 0.35) (layer "F.Cu") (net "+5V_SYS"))
 (segment (start 34.94 60) (end 35.94 57) (width 0.65) (layer "F.Cu") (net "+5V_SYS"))
 (segment (start 50 84.5) (end 50 85.5875) (width 0.35) (layer "F.Cu") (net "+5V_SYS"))
 (segment (start 51 89) (end 50.5 89) (width 0.24) (layer "F.Cu") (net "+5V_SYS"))
 (segment (start 43.54 36) (end 43.54 34) (width 0.5) (layer "F.Cu") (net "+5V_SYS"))
 (via (at 58 36) (size 0.8) (drill 0.4) (layers "F.Cu" "B.Cu") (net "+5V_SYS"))
 (via (at 58 18.16) (size 0.8) (drill 0.4) (layers "F.Cu" "B.Cu") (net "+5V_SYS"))
 (via (at 58 57) (size 0.8) (drill 0.4) (layers "F.Cu" "B.Cu") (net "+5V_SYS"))
 (via (at 58 84.5) (size 0.8) (drill 0.4) (layers "F.Cu" "B.Cu") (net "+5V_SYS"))
 (segment (start 50 119) (end 58 119) (width 0.9) (layer "B.Cu") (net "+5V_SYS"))
 (segment (start 58 119) (end 58 18.16) (width 0.9) (layer "B.Cu") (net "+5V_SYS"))
 (segment (start 52 50) (end 54.0875 50) (width 0.28) (layer "F.Cu") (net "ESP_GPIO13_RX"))
 (segment (start 46.9125 50) (end 52 50) (width 0.28) (layer "F.Cu") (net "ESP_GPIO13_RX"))
 (via (at 52 50) (size 0.8) (drill 0.4) (layers "F.Cu" "B.Cu") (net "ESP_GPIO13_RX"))
 (segment (start 52 15.62) (end 42 15.62) (width 0.28) (layer "B.Cu") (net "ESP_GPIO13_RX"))
 (segment (start 52 50) (end 52 15.62) (width 0.28) (layer "B.Cu") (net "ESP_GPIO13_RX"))
 (segment (start 50 43) (end 50 45) (width 0.28) (layer "F.Cu") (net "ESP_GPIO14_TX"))
 (segment (start 50 45) (end 46.9125 45) (width 0.28) (layer "F.Cu") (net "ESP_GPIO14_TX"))
 (via (at 50 43) (size 0.8) (drill 0.4) (layers "F.Cu" "B.Cu") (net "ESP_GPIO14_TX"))
 (segment (start 39.5 43) (end 50 43) (width 0.28) (layer "B.Cu") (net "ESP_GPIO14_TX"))
 (segment (start 42 20.7) (end 39.5 20.7) (width 0.28) (layer "B.Cu") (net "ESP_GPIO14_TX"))
 (segment (start 39.5 20.7) (end 39.5 43) (width 0.28) (layer "B.Cu") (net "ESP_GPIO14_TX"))
 (segment (start 46.08 28) (end 46.08 34) (width 0.28) (layer "F.Cu") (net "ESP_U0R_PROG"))
 (segment (start 61 28) (end 46.08 28) (width 0.28) (layer "F.Cu") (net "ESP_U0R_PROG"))
 (segment (start 61 20.7) (end 61 28) (width 0.28) (layer "F.Cu") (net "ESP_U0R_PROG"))
 (segment (start 64.86 20.7) (end 61 20.7) (width 0.28) (layer "F.Cu") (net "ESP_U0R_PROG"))
 (segment (start 63.5 31.5) (end 48.62 31.5) (width 0.28) (layer "F.Cu") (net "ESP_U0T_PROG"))
 (segment (start 64.86 23.24) (end 63.5 23.24) (width 0.28) (layer "F.Cu") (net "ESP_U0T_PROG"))
 (segment (start 63.5 23.24) (end 63.5 31.5) (width 0.28) (layer "F.Cu") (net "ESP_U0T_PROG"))
 (segment (start 48.62 31.5) (end 48.62 34) (width 0.28) (layer "F.Cu") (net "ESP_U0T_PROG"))
 (segment (start 64.86 13.08) (end 60.5 13.08) (width 0.28) (layer "B.Cu") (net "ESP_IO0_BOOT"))
 (segment (start 60.5 13.08) (end 60.5 39) (width 0.28) (layer "B.Cu") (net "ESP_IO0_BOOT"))
 (segment (start 60.5 39) (end 61 39) (width 0.28) (layer "B.Cu") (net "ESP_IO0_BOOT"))
 (segment (start 33.4 72) (end 41.3 72) (width 0.28) (layer "F.Cu") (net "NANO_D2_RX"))
 (segment (start 41.3 45) (end 45.0875 45) (width 0.28) (layer "F.Cu") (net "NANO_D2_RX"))
 (via (at 41.3 45) (size 0.8) (drill 0.4) (layers "F.Cu" "B.Cu") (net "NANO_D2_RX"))
 (via (at 33.4 72) (size 0.8) (drill 0.4) (layers "F.Cu" "B.Cu") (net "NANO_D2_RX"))
 (via (at 41.3 72) (size 0.8) (drill 0.4) (layers "F.Cu" "B.Cu") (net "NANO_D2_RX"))
 (segment (start 32.4 75.24) (end 33.4 72) (width 0.28) (layer "B.Cu") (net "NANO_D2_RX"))
 (segment (start 41.3 72) (end 41.3 45) (width 0.28) (layer "B.Cu") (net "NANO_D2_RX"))
 (segment (start 38.75 50) (end 45.0875 50) (width 0.28) (layer "F.Cu") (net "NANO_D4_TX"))
 (via (at 38.75 50) (size 0.8) (drill 0.4) (layers "F.Cu" "B.Cu") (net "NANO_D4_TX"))
 (segment (start 38.75 80) (end 38.75 50) (width 0.28) (layer "B.Cu") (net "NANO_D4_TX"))
 (segment (start 28.32 80) (end 38.75 80) (width 0.28) (layer "B.Cu") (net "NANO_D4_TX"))
 (segment (start 27.32 75.24) (end 28.32 80) (width 0.28) (layer "B.Cu") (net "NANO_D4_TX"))
 (segment (start 55 82) (end 61.0875 82) (width 0.24) (layer "F.Cu") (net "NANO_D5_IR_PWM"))
 (via (at 55 82) (size 0.8) (drill 0.4) (layers "F.Cu" "B.Cu") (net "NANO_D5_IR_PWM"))
 (segment (start 24.78 82) (end 55 82) (width 0.28) (layer "B.Cu") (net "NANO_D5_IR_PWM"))
 (segment (start 24.78 75.24) (end 24.78 82) (width 0.28) (layer "B.Cu") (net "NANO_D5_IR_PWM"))
 (segment (start 36 84) (end 37.0875 82) (width 0.24) (layer "F.Cu") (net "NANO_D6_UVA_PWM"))
 (via (at 36 84) (size 0.8) (drill 0.4) (layers "F.Cu" "B.Cu") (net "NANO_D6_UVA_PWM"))
 (segment (start 22.24 75.24) (end 22.24 84) (width 0.28) (layer "B.Cu") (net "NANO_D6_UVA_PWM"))
 (segment (start 22.24 84) (end 36 84) (width 0.28) (layer "B.Cu") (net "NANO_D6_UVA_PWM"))
 (segment (start 48 86) (end 49.0875 80) (width 0.28) (layer "F.Cu") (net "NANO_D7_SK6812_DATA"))
 (via (at 48 86) (size 0.8) (drill 0.4) (layers "F.Cu" "B.Cu") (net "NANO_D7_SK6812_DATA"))
 (segment (start 19.7 86) (end 48 86) (width 0.28) (layer "B.Cu") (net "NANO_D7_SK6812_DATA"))
 (segment (start 19.7 75.24) (end 19.7 86) (width 0.28) (layer "B.Cu") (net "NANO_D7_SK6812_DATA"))
 (segment (start 66.8 91.95) (end 63.9375 91.95) (width 0.24) (layer "F.Cu") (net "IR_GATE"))
 (segment (start 66.8 86.2) (end 66.8 91.95) (width 0.24) (layer "F.Cu") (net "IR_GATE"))
 (segment (start 62.9125 82) (end 63 86.2) (width 0.24) (layer "F.Cu") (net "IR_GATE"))
 (segment (start 62.9125 85) (end 63 86.2) (width 0.24) (layer "F.Cu") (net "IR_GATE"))
 (segment (start 63 86.2) (end 66.8 86.2) (width 0.24) (layer "F.Cu") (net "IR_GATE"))
 (segment (start 40 86.2) (end 45.06 86.2) (width 0.24) (layer "F.Cu") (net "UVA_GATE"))
 (segment (start 45.06 86.2) (end 45.0625 90.05) (width 0.24) (layer "F.Cu") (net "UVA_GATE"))
 (segment (start 38.9125 85) (end 40 86.2) (width 0.24) (layer "F.Cu") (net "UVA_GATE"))
 (segment (start 38.9125 82) (end 40 86.2) (width 0.24) (layer "F.Cu") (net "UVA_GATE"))
 (segment (start 62.0625 91) (end 57.5 91) (width 0.24) (layer "F.Cu") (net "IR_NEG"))
 (segment (start 57.5 91) (end 58.125 94.15) (width 0.24) (layer "F.Cu") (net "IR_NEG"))
 (segment (start 48.5 91) (end 46.875 94.15) (width 0.24) (layer "F.Cu") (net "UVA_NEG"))
 (segment (start 46.9375 91) (end 48.5 91) (width 0.24) (layer "F.Cu") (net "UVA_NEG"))
 (segment (start 58 87.4125) (end 56.5 88) (width 0.24) (layer "F.Cu") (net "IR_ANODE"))
 (segment (start 56.5 88) (end 56.875 94.15) (width 0.24) (layer "F.Cu") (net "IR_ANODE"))
 (segment (start 50 87.4125) (end 49.5 89.5) (width 0.24) (layer "F.Cu") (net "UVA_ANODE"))
 (segment (start 49.5 89.5) (end 48.125 94.15) (width 0.24) (layer "F.Cu") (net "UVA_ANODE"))
 (segment (start 54.5 93.6) (end 54.375 94.15) (width 0.2) (layer "F.Cu") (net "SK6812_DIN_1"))
 (segment (start 50.9125 80) (end 52 80) (width 0.2) (layer "F.Cu") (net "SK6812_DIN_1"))
 (via (at 54.5 93.6) (size 0.8) (drill 0.4) (layers "F.Cu" "B.Cu") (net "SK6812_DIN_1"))
 (via (at 52 80) (size 0.8) (drill 0.4) (layers "F.Cu" "B.Cu") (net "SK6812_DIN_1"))
 (segment (start 52 80) (end 56.5 80) (width 0.2) (layer "B.Cu") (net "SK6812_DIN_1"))
 (segment (start 54.5 86) (end 54.5 93.6) (width 0.2) (layer "B.Cu") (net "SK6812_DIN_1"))
 (segment (start 56.5 80) (end 56.5 86) (width 0.2) (layer "B.Cu") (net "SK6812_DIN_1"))
 (segment (start 56.5 86) (end 54.5 86) (width 0.2) (layer "B.Cu") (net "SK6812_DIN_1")))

